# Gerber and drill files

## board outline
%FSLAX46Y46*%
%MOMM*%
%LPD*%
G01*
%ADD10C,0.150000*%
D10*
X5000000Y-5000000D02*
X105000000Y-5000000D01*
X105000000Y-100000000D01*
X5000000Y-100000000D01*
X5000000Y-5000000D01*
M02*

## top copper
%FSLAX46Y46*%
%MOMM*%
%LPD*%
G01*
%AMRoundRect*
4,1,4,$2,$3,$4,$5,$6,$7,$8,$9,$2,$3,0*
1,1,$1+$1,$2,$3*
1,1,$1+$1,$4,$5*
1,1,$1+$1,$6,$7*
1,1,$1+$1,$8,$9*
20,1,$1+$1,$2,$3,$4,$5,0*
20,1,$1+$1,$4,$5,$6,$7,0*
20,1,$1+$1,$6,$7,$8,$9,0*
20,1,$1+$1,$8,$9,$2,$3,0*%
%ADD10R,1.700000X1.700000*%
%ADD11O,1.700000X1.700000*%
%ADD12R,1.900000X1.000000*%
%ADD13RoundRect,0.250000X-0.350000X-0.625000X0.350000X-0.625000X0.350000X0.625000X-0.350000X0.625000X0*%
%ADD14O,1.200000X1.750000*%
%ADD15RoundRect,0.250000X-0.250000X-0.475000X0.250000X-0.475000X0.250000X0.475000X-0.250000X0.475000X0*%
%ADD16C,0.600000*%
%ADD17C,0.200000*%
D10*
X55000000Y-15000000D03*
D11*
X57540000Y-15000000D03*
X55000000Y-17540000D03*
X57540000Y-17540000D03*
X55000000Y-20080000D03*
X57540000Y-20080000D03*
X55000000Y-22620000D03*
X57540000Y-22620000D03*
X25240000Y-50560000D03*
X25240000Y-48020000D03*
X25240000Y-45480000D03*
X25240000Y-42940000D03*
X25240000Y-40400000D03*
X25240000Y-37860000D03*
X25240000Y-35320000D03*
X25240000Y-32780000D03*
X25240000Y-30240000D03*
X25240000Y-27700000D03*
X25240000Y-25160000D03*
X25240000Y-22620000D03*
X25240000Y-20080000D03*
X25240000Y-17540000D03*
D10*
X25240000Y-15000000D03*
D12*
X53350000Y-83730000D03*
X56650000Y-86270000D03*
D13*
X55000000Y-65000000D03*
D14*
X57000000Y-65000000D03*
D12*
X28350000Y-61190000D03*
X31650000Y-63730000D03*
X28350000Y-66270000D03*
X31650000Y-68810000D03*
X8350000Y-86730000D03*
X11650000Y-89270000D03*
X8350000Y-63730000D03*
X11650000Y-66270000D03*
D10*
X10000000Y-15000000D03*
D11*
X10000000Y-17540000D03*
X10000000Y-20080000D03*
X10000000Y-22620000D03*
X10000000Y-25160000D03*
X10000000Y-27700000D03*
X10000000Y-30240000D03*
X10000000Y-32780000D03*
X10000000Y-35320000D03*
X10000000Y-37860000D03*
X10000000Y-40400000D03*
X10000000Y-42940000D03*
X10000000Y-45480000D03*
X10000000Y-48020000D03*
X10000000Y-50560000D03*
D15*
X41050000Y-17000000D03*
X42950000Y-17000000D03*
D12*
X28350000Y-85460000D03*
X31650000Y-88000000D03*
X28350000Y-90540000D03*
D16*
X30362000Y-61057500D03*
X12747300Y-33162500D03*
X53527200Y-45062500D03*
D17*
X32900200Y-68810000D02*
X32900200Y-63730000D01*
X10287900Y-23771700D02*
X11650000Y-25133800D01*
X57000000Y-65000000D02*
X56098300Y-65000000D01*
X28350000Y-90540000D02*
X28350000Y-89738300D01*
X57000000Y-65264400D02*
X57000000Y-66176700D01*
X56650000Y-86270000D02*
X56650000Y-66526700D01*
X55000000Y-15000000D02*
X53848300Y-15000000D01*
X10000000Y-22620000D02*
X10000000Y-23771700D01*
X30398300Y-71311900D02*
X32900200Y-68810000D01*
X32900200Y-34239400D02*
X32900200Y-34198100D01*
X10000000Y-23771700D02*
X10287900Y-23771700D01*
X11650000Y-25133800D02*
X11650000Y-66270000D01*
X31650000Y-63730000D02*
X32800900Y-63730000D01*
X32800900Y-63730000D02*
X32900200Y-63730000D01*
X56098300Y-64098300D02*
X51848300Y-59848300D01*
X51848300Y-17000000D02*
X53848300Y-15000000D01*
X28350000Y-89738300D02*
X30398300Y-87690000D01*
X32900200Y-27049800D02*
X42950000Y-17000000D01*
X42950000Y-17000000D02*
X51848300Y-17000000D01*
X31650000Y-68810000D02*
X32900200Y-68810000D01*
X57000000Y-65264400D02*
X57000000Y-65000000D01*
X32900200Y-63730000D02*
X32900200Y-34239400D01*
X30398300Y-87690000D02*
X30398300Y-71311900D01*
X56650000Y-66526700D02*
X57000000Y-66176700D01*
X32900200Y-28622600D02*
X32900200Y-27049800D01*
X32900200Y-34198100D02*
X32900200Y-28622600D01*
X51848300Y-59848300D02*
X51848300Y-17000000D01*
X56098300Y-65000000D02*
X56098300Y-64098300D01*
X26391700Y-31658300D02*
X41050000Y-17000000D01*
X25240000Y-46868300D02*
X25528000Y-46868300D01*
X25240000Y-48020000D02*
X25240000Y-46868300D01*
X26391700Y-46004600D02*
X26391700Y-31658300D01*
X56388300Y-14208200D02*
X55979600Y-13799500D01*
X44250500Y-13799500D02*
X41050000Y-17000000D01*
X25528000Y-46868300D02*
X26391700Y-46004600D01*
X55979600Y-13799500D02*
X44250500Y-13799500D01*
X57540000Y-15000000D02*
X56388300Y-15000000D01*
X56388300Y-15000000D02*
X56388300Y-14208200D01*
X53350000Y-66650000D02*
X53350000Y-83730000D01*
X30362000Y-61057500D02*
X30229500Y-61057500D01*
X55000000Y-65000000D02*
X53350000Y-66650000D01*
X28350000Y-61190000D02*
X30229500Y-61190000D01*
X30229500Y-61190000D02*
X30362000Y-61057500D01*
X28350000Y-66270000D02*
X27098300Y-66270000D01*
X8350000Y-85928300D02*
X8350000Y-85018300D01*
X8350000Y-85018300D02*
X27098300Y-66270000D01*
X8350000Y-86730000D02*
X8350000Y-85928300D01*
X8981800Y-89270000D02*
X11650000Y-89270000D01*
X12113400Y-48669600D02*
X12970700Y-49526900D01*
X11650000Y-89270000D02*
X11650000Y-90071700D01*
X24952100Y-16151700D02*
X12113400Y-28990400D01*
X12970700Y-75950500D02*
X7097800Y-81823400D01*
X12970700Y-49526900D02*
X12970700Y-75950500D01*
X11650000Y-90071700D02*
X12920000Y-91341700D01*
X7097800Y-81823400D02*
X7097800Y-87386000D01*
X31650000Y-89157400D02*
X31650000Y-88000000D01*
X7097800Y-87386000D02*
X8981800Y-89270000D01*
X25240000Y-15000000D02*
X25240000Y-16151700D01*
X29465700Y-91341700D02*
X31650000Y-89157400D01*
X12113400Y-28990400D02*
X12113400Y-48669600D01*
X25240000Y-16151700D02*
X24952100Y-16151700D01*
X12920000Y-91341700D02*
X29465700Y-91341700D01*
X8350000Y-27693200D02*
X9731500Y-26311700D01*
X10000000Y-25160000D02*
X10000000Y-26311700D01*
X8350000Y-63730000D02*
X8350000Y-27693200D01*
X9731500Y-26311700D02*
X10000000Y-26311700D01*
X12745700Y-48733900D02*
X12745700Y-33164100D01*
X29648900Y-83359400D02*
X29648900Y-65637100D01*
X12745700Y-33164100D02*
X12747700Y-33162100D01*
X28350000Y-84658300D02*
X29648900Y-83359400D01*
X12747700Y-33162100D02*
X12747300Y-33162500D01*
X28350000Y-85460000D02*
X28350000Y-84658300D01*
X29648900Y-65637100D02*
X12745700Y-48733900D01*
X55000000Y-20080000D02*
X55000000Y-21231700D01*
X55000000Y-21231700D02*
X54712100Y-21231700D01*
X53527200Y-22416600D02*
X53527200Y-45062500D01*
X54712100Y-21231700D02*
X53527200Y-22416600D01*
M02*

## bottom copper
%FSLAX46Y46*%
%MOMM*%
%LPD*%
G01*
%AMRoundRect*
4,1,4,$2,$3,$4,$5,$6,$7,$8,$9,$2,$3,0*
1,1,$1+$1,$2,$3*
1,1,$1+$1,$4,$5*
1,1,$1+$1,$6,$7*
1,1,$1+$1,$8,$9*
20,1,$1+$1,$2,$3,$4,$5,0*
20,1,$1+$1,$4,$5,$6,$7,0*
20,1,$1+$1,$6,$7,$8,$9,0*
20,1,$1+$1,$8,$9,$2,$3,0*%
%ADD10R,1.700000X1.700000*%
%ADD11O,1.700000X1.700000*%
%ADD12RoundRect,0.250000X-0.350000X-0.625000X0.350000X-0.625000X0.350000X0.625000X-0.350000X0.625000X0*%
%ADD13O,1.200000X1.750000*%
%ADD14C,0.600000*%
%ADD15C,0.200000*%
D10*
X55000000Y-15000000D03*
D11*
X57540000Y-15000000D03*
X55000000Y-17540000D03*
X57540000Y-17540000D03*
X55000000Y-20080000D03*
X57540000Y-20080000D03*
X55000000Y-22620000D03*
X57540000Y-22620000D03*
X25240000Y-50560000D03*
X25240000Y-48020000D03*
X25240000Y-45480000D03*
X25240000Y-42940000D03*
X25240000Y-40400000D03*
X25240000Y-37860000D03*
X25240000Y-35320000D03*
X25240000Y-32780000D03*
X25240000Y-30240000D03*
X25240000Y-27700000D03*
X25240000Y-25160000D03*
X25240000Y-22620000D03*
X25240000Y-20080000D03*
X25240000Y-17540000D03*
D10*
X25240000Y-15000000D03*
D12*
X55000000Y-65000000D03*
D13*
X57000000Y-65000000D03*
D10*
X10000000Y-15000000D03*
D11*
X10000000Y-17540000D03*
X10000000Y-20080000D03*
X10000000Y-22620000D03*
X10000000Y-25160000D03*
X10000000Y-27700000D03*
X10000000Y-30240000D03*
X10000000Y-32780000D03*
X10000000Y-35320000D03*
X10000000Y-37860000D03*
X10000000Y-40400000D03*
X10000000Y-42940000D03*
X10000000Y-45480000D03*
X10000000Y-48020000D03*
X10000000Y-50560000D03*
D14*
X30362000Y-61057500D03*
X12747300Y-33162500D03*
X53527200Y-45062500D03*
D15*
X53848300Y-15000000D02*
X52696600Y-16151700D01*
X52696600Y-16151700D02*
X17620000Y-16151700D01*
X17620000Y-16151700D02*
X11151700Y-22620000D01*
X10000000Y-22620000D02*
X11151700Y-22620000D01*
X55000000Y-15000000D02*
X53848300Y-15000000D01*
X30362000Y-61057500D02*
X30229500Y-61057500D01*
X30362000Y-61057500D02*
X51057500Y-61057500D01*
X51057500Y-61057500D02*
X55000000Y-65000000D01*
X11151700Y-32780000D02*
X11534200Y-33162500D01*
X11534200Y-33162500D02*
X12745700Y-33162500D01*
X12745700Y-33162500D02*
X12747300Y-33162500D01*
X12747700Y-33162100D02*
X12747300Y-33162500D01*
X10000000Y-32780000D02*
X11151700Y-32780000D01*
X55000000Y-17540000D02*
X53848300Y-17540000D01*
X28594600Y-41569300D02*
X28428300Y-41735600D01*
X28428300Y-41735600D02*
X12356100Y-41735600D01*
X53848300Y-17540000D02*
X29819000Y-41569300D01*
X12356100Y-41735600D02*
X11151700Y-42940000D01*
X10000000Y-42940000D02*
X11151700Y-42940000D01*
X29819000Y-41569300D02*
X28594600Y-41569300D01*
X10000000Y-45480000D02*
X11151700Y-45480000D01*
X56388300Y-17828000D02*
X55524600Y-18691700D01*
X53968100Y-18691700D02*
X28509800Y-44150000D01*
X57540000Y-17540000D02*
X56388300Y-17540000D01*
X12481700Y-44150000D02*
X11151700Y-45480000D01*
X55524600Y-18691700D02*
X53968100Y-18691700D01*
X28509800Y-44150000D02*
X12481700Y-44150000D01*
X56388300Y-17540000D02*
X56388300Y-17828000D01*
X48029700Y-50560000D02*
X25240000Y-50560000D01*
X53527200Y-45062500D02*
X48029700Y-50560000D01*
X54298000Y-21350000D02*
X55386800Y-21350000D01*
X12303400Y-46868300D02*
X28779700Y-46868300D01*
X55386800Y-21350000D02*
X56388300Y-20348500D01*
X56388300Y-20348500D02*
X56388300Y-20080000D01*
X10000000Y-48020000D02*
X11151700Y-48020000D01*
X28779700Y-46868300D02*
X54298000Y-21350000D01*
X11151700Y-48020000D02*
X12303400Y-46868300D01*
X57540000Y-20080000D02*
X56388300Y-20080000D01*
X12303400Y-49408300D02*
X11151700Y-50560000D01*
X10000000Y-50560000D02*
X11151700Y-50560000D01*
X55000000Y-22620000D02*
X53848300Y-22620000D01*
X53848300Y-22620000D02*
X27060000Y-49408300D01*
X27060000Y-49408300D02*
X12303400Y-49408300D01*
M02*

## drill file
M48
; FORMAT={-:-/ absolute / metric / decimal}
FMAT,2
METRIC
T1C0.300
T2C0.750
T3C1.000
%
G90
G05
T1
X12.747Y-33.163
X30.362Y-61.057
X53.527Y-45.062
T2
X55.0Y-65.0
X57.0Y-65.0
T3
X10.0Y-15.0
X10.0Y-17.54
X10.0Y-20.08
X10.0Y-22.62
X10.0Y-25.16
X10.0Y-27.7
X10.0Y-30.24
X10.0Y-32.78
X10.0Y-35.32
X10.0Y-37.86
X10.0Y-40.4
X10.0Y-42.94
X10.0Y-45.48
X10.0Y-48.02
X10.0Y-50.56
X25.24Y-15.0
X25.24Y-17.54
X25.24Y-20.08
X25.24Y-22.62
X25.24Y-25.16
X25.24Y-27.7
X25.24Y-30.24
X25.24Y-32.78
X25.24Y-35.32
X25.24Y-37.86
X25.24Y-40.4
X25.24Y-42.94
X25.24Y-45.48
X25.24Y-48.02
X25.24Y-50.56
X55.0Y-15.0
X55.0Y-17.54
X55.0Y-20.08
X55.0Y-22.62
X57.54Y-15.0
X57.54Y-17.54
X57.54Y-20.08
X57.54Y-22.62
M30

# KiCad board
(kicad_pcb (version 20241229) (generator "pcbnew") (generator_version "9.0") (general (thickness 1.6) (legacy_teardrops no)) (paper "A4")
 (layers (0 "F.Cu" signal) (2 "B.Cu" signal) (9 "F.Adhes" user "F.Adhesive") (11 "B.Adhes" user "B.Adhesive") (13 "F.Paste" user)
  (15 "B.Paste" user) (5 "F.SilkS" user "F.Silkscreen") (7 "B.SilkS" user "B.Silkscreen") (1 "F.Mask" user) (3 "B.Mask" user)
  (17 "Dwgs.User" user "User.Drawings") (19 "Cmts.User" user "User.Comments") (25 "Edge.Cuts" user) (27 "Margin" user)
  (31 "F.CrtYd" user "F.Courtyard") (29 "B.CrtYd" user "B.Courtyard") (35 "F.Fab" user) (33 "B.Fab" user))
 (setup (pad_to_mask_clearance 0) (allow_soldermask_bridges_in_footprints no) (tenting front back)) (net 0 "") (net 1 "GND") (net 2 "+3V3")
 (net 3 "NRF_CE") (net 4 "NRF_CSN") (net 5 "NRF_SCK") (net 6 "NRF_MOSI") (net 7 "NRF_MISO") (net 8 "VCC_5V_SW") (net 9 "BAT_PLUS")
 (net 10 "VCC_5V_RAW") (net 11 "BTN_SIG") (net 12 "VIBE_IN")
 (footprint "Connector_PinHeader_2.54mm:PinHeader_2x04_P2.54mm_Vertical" (layer "F.Cu") (at 55 15)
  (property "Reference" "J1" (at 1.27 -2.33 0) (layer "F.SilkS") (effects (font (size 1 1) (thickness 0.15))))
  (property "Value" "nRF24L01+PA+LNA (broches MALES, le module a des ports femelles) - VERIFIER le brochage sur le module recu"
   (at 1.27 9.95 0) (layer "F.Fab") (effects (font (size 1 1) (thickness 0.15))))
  (pad "1" thru_hole rect (at 0 0) (size 1.7 1.7) (drill 1) (layers "*.Cu" "*.Mask") (remove_unused_layers no) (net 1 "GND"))
  (pad "2" thru_hole oval (at 2.54 0) (size 1.7 1.7) (drill 1) (layers "*.Cu" "*.Mask") (remove_unused_layers no) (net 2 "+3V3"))
  (pad "3" thru_hole oval (at 0 2.54) (size 1.7 1.7) (drill 1) (layers "*.Cu" "*.Mask") (remove_unused_layers no) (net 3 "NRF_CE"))
  (pad "4" thru_hole oval (at 2.54 2.54) (size 1.7 1.7) (drill 1) (layers "*.Cu" "*.Mask") (remove_unused_layers no) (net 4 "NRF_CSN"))
  (pad "5" thru_hole oval (at 0 5.08) (size 1.7 1.7) (drill 1) (layers "*.Cu" "*.Mask") (remove_unused_layers no) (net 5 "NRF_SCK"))
  (pad "6" thru_hole oval (at 2.54 5.08) (size 1.7 1.7) (drill 1) (layers "*.Cu" "*.Mask") (remove_unused_layers no) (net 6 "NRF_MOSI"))
  (pad "7" thru_hole oval (at 0 7.62) (size 1.7 1.7) (drill 1) (layers "*.Cu" "*.Mask") (remove_unused_layers no) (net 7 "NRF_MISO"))
  (pad "8" thru_hole oval (at 2.54 7.62) (size 1.7 1.7) (drill 1) (layers "*.Cu" "*.Mask") (remove_unused_layers no)))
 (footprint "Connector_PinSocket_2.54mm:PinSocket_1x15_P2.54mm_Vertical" (layer "F.Cu") (at 25.24 15)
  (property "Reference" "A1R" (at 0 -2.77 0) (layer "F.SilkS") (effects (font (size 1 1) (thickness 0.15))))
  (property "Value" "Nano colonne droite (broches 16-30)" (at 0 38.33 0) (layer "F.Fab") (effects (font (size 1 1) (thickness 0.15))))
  (pad "16" thru_hole oval (at 0 35.56) (size 1.7 1.7) (drill 1) (layers "*.Cu" "*.Mask") (remove_unused_layers no) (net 5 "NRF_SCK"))
  (pad "17" thru_hole oval (at 0 33.02) (size 1.7 1.7) (drill 1) (layers "*.Cu" "*.Mask") (remove_unused_layers no) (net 2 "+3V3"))
  (pad "18" thru_hole oval (at 0 30.48) (size 1.7 1.7) (drill 1) (layers "*.Cu" "*.Mask") (remove_unused_layers no))
  (pad "19" thru_hole oval (at 0 27.94) (size 1.7 1.7) (drill 1) (layers "*.Cu" "*.Mask") (remove_unused_layers no))
  (pad "20" thru_hole oval (at 0 25.4) (size 1.7 1.7) (drill 1) (layers "*.Cu" "*.Mask") (remove_unused_layers no))
  (pad "21" thru_hole oval (at 0 22.86) (size 1.7 1.7) (drill 1) (layers "*.Cu" "*.Mask") (remove_unused_layers no))
  (pad "22" thru_hole oval (at 0 20.32) (size 1.7 1.7) (drill 1) (layers "*.Cu" "*.Mask") (remove_unused_layers no))
  (pad "23" thru_hole oval (at 0 17.78) (size 1.7 1.7) (drill 1) (layers "*.Cu" "*.Mask") (remove_unused_layers no))
  (pad "24" thru_hole oval (at 0 15.24) (size 1.7 1.7) (drill 1) (layers "*.Cu" "*.Mask") (remove_unused_layers no))
  (pad "25" thru_hole oval (at 0 12.7) (size 1.7 1.7) (drill 1) (layers "*.Cu" "*.Mask") (remove_unused_layers no))
  (pad "26" thru_hole oval (at 0 10.16) (size 1.7 1.7) (drill 1) (layers "*.Cu" "*.Mask") (remove_unused_layers no))
  (pad "27" thru_hole oval (at 0 7.62) (size 1.7 1.7) (drill 1) (layers "*.Cu" "*.Mask") (remove_unused_layers no))
  (pad "28" thru_hole oval (at 0 5.08) (size 1.7 1.7) (drill 1) (layers "*.Cu" "*.Mask") (remove_unused_layers no))
  (pad "29" thru_hole oval (at 0 2.54) (size 1.7 1.7) (drill 1) (layers "*.Cu" "*.Mask") (remove_unused_layers no))
  (pad "30" thru_hole rect (at 0 0) (size 1.7 1.7) (drill 1) (layers "*.Cu" "*.Mask") (remove_unused_layers no) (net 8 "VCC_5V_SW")))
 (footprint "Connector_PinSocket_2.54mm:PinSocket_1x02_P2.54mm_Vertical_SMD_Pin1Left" (layer "F.Cu") (at 55 85)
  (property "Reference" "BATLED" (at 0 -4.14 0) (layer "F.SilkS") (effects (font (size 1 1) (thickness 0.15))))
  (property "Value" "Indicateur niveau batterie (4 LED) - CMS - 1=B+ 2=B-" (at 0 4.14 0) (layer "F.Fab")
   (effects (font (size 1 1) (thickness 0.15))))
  (pad "1" smd rect (at -1.65 -1.27) (size 1.9 1) (layers "F.Cu" "F.Mask" "F.Paste") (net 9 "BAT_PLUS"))
  (pad "2" smd rect (at 1.65 1.27) (size 1.9 1) (layers "F.Cu" "F.Mask" "F.Paste") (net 1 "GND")))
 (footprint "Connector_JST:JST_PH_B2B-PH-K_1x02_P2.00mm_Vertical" (layer "F.Cu") (at 55 65)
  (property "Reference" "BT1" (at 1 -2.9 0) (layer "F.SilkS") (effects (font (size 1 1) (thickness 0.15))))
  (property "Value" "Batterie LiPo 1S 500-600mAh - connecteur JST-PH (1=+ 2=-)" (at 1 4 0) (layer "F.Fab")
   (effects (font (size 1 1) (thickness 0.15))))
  (pad "1" thru_hole roundrect (at 0 0) (size 1.2 1.75) (drill 0.75) (layers "*.Cu" "*.Mask") (remove_unused_layers no)
   (roundrect_rratio 0.208333) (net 9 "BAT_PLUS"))
  (pad "2" thru_hole oval (at 2 0) (size 1.2 1.75) (drill 0.75) (layers "*.Cu" "*.Mask") (remove_unused_layers no) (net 1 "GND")))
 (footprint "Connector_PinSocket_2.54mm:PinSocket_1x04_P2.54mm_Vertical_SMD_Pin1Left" (layer "F.Cu") (at 30 65)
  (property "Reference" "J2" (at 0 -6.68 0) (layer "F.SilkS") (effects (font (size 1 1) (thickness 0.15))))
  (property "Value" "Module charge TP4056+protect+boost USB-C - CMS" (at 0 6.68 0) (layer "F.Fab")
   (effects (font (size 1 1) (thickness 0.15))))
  (pad "1" smd rect (at -1.65 -3.81) (size 1.9 1) (layers "F.Cu" "F.Mask" "F.Paste") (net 9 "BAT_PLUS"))
  (pad "2" smd rect (at 1.65 -1.27) (size 1.9 1) (layers "F.Cu" "F.Mask" "F.Paste") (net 1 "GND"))
  (pad "3" smd rect (at -1.65 1.27) (size 1.9 1) (layers "F.Cu" "F.Mask" "F.Paste") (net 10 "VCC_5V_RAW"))
  (pad "4" smd rect (at 1.65 3.81) (size 1.9 1) (layers "F.Cu" "F.Mask" "F.Paste") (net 1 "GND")))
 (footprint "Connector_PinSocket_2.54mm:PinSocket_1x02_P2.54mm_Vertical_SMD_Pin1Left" (layer "F.Cu") (at 10 88)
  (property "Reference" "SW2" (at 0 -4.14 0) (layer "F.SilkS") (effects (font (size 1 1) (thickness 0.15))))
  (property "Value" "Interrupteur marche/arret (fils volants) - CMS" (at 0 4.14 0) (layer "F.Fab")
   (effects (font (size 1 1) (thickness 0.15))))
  (pad "1" smd rect (at -1.65 -1.27) (size 1.9 1) (layers "F.Cu" "F.Mask" "F.Paste") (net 10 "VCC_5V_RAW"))
  (pad "2" smd rect (at 1.65 1.27) (size 1.9 1) (layers "F.Cu" "F.Mask" "F.Paste") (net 8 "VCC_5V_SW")))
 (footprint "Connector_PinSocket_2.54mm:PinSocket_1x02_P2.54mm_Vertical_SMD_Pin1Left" (layer "F.Cu") (at 10 65)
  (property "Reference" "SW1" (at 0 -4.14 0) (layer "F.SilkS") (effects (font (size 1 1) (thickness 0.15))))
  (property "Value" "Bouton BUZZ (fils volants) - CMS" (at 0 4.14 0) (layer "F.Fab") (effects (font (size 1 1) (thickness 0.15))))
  (pad "1" smd rect (at -1.65 -1.27) (size 1.9 1) (layers "F.Cu" "F.Mask" "F.Paste") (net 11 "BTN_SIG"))
  (pad "2" smd rect (at 1.65 1.27) (size 1.9 1) (layers "F.Cu" "F.Mask" "F.Paste") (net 1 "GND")))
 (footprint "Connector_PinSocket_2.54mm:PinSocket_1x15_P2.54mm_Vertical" (layer "F.Cu") (at 10 15)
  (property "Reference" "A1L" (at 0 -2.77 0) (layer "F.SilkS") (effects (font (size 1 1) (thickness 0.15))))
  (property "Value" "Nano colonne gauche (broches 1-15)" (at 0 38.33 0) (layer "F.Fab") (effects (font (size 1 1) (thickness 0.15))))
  (pad "1" thru_hole rect (at 0 0) (size 1.7 1.7) (drill 1) (layers "*.Cu" "*.Mask") (remove_unused_layers no))
  (pad "2" thru_hole oval (at 0 2.54) (size 1.7 1.7) (drill 1) (layers "*.Cu" "*.Mask") (remove_unused_layers no))
  (pad "3" thru_hole oval (at 0 5.08) (size 1.7 1.7) (drill 1) (layers "*.Cu" "*.Mask") (remove_unused_layers no))
  (pad "4" thru_hole oval (at 0 7.62) (size 1.7 1.7) (drill 1) (layers "*.Cu" "*.Mask") (remove_unused_layers no) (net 1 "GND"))
  (pad "5" thru_hole oval (at 0 10.16) (size 1.7 1.7) (drill 1) (layers "*.Cu" "*.Mask") (remove_unused_layers no) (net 11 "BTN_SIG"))
  (pad "6" thru_hole oval (at 0 12.7) (size 1.7 1.7) (drill 1) (layers "*.Cu" "*.Mask") (remove_unused_layers no))
  (pad "7" thru_hole oval (at 0 15.24) (size 1.7 1.7) (drill 1) (layers "*.Cu" "*.Mask") (remove_unused_layers no))
  (pad "8" thru_hole oval (at 0 17.78) (size 1.7 1.7) (drill 1) (layers "*.Cu" "*.Mask") (remove_unused_layers no) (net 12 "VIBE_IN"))
  (pad "9" thru_hole oval (at 0 20.32) (size 1.7 1.7) (drill 1) (layers "*.Cu" "*.Mask") (remove_unused_layers no))
  (pad "10" thru_hole oval (at 0 22.86) (size 1.7 1.7) (drill 1) (layers "*.Cu" "*.Mask") (remove_unused_layers no))
  (pad "11" thru_hole oval (at 0 25.4) (size 1.7 1.7) (drill 1) (layers "*.Cu" "*.Mask") (remove_unused_layers no))
  (pad "12" thru_hole oval (at 0 27.94) (size 1.7 1.7) (drill 1) (layers "*.Cu" "*.Mask") (remove_unused_layers no) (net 3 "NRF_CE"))
  (pad "13" thru_hole oval (at 0 30.48) (size 1.7 1.7) (drill 1) (layers "*.Cu" "*.Mask") (remove_unused_layers no) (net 4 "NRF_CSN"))
  (pad "14" thru_hole oval (at 0 33.02) (size 1.7 1.7) (drill 1) (layers "*.Cu" "*.Mask") (remove_unused_layers no) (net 6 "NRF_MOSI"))
  (pad "15" thru_hole oval (at 0 35.56) (size 1.7 1.7) (drill 1) (layers "*.Cu" "*.Mask") (remove_unused_layers no) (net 7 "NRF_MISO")))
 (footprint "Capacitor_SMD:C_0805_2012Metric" (layer "F.Cu") (at 42 17)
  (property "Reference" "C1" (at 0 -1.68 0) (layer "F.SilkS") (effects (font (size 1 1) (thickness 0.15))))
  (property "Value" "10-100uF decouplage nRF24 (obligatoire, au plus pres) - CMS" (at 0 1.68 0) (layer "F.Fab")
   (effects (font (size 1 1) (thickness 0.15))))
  (pad "1" smd roundrect (at -0.95 0) (size 1 1.45) (layers "F.Cu" "F.Mask" "F.Paste") (roundrect_rratio 0.25) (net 2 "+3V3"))
  (pad "2" smd roundrect (at 0.95 0) (size 1 1.45) (layers "F.Cu" "F.Mask" "F.Paste") (roundrect_rratio 0.25) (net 1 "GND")))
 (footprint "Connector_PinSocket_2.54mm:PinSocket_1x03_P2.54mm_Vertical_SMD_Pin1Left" (layer "F.Cu") (at 30 88)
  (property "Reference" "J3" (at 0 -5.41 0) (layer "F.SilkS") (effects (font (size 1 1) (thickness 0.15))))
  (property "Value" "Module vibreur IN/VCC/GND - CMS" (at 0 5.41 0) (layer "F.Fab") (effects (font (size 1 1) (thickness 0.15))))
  (pad "1" smd rect (at -1.65 -2.54) (size 1.9 1) (layers "F.Cu" "F.Mask" "F.Paste") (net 12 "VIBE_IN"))
  (pad "2" smd rect (at 1.65 0) (size 1.9 1) (layers "F.Cu" "F.Mask" "F.Paste") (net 8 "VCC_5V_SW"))
  (pad "3" smd rect (at -1.65 2.54) (size 1.9 1) (layers "F.Cu" "F.Mask" "F.Paste") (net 1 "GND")))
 (gr_rect (start 5 5) (end 105 100) (stroke (width 0.15) (type default)) (fill no) (layer "Edge.Cuts"))
 (segment (start 32.9002 68.81) (end 32.9002 63.73) (width 0.2) (layer "F.Cu") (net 1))
 (segment (start 10.2879 23.7717) (end 11.65 25.1338) (width 0.2) (layer "F.Cu") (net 1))
 (segment (start 57 65) (end 56.0983 65) (width 0.2) (layer "F.Cu") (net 1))
 (segment (start 28.35 90.54) (end 28.35 89.7383) (width 0.2) (layer "F.Cu") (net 1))
 (segment (start 57 65.2644) (end 57 66.1767) (width 0.2) (layer "F.Cu") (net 1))
 (segment (start 56.65 86.27) (end 56.65 66.5267) (width 0.2) (layer "F.Cu") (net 1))
 (segment (start 55 15) (end 53.8483 15) (width 0.2) (layer "F.Cu") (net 1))
 (segment (start 10 22.62) (end 10 23.7717) (width 0.2) (layer "F.Cu") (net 1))
 (segment (start 30.3983 71.3119) (end 32.9002 68.81) (width 0.2) (layer "F.Cu") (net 1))
 (segment (start 32.9002 34.2394) (end 32.9002 34.1981) (width 0.2) (layer "F.Cu") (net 1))
 (segment (start 10 23.7717) (end 10.2879 23.7717) (width 0.2) (layer "F.Cu") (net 1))
 (segment (start 11.65 25.1338) (end 11.65 66.27) (width 0.2) (layer "F.Cu") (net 1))
 (segment (start 31.65 63.73) (end 32.8009 63.73) (width 0.2) (layer "F.Cu") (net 1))
 (segment (start 32.8009 63.73) (end 32.9002 63.73) (width 0.2) (layer "F.Cu") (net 1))
 (segment (start 56.0983 64.0983) (end 51.8483 59.8483) (width 0.2) (layer "F.Cu") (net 1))
 (segment (start 51.8483 17) (end 53.8483 15) (width 0.2) (layer "F.Cu") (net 1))
 (segment (start 28.35 89.7383) (end 30.3983 87.69) (width 0.2) (layer "F.Cu") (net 1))
 (segment (start 32.9002 27.0498) (end 42.95 17) (width 0.2) (layer "F.Cu") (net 1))
 (segment (start 42.95 17) (end 51.8483 17) (width 0.2) (layer "F.Cu") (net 1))
 (segment (start 31.65 68.81) (end 32.9002 68.81) (width 0.2) (layer "F.Cu") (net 1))
 (segment (start 57 65.2644) (end 57 65) (width 0.2) (layer "F.Cu") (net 1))
 (segment (start 32.9002 63.73) (end 32.9002 34.2394) (width 0.2) (layer "F.Cu") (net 1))
 (segment (start 30.3983 87.69) (end 30.3983 71.3119) (width 0.2) (layer "F.Cu") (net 1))
 (segment (start 56.65 66.5267) (end 57 66.1767) (width 0.2) (layer "F.Cu") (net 1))
 (segment (start 32.9002 28.6226) (end 32.9002 27.0498) (width 0.2) (layer "F.Cu") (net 1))
 (segment (start 32.9002 34.1981) (end 32.9002 28.6226) (width 0.2) (layer "F.Cu") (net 1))
 (segment (start 51.8483 59.8483) (end 51.8483 17) (width 0.2) (layer "F.Cu") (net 1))
 (segment (start 56.0983 65) (end 56.0983 64.0983) (width 0.2) (layer "F.Cu") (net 1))
 (segment (start 53.8483 15) (end 52.6966 16.1517) (width 0.2) (layer "B.Cu") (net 1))
 (segment (start 52.6966 16.1517) (end 17.62 16.1517) (width 0.2) (layer "B.Cu") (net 1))
 (segment (start 17.62 16.1517) (end 11.1517 22.62) (width 0.2) (layer "B.Cu") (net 1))
 (segment (start 10 22.62) (end 11.1517 22.62) (width 0.2) (layer "B.Cu") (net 1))
 (segment (start 55 15) (end 53.8483 15) (width 0.2) (layer "B.Cu") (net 1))
 (segment (start 26.3917 31.6583) (end 41.05 17) (width 0.2) (layer "F.Cu") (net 2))
 (segment (start 25.24 46.8683) (end 25.528 46.8683) (width 0.2) (layer "F.Cu") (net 2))
 (segment (start 25.24 48.02) (end 25.24 46.8683) (width 0.2) (layer "F.Cu") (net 2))
 (segment (start 26.3917 46.0046) (end 26.3917 31.6583) (width 0.2) (layer "F.Cu") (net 2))
 (segment (start 56.3883 14.2082) (end 55.9796 13.7995) (width 0.2) (layer "F.Cu") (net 2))
 (segment (start 44.2505 13.7995) (end 41.05 17) (width 0.2) (layer "F.Cu") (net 2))
 (segment (start 25.528 46.8683) (end 26.3917 46.0046) (width 0.2) (layer "F.Cu") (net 2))
 (segment (start 55.9796 13.7995) (end 44.2505 13.7995) (width 0.2) (layer "F.Cu") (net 2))
 (segment (start 57.54 15) (end 56.3883 15) (width 0.2) (layer "F.Cu") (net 2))
 (segment (start 56.3883 15) (end 56.3883 14.2082) (width 0.2) (layer "F.Cu") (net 2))
 (segment (start 53.35 66.65) (end 53.35 83.73) (width 0.2) (layer "F.Cu") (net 9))
 (segment (start 30.362 61.0575) (end 30.2295 61.0575) (width 0.2) (layer "F.Cu") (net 9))
 (segment (start 55 65) (end 53.35 66.65) (width 0.2) (layer "F.Cu") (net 9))
 (segment (start 28.35 61.19) (end 30.2295 61.19) (width 0.2) (layer "F.Cu") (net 9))
 (segment (start 30.2295 61.19) (end 30.362 61.0575) (width 0.2) (layer "F.Cu") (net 9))
 (via (at 30.362 61.0575) (size 0.6) (drill 0.3) (layers "F.Cu" "B.Cu") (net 9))
 (segment (start 30.362 61.0575) (end 30.2295 61.0575) (width 0.2) (layer "B.Cu") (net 9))
 (segment (start 30.362 61.0575) (end 51.0575 61.0575) (width 0.2) (layer "B.Cu") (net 9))
 (segment (start 51.0575 61.0575) (end 55 65) (width 0.2) (layer "B.Cu") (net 9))
 (segment (start 28.35 66.27) (end 27.0983 66.27) (width 0.2) (layer "F.Cu") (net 10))
 (segment (start 8.35 85.9283) (end 8.35 85.0183) (width 0.2) (layer "F.Cu") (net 10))
 (segment (start 8.35 85.0183) (end 27.0983 66.27) (width 0.2) (layer "F.Cu") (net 10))
 (segment (start 8.35 86.73) (end 8.35 85.9283) (width 0.2) (layer "F.Cu") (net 10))
 (segment (start 8.9818 89.27) (end 11.65 89.27) (width 0.2) (layer "F.Cu") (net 8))
 (segment (start 12.1134 48.6696) (end 12.9707 49.5269) (width 0.2) (layer "F.Cu") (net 8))
 (segment (start 11.65 89.27) (end 11.65 90.0717) (width 0.2) (layer "F.Cu") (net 8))
 (segment (start 24.9521 16.1517) (end 12.1134 28.9904) (width 0.2) (layer "F.Cu") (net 8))
 (segment (start 12.9707 75.9505) (end 7.0978 81.8234) (width 0.2) (layer "F.Cu") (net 8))
 (segment (start 12.9707 49.5269) (end 12.9707 75.9505) (width 0.2) (layer "F.Cu") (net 8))
 (segment (start 11.65 90.0717) (end 12.92 91.3417) (width 0.2) (layer "F.Cu") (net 8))
 (segment (start 7.0978 81.8234) (end 7.0978 87.386) (width 0.2) (layer "F.Cu") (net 8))
 (segment (start 31.65 89.1574) (end 31.65 88) (width 0.2) (layer "F.Cu") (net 8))
 (segment (start 7.0978 87.386) (end 8.9818 89.27) (width 0.2) (layer "F.Cu") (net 8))
 (segment (start 25.24 15) (end 25.24 16.1517) (width 0.2) (layer "F.Cu") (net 8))
 (segment (start 29.4657 91.3417) (end 31.65 89.1574) (width 0.2) (layer "F.Cu") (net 8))
 (segment (start 12.1134 28.9904) (end 12.1134 48.6696) (width 0.2) (layer "F.Cu") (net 8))
 (segment (start 25.24 16.1517) (end 24.9521 16.1517) (width 0.2) (layer "F.Cu") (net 8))
 (segment (start 12.92 91.3417) (end 29.4657 91.3417) (width 0.2) (layer "F.Cu") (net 8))
 (segment (start 8.35 27.6932) (end 9.7315 26.3117) (width 0.2) (layer "F.Cu") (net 11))
 (segment (start 10 25.16) (end 10 26.3117) (width 0.2) (layer "F.Cu") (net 11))
 (segment (start 8.35 63.73) (end 8.35 27.6932) (width 0.2) (layer "F.Cu") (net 11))
 (segment (start 9.7315 26.3117) (end 10 26.3117) (width 0.2) (layer "F.Cu") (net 11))
 (segment (start 12.7457 48.7339) (end 12.7457 33.1641) (width 0.2) (layer "F.Cu") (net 12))
 (segment (start 29.6489 83.3594) (end 29.6489 65.6371) (width 0.2) (layer "F.Cu") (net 12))
 (segment (start 12.7457 33.1641) (end 12.7477 33.1621) (width 0.2) (layer "F.Cu") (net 12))
 (segment (start 28.35 84.6583) (end 29.6489 83.3594) (width 0.2) (layer "F.Cu") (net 12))
 (segment (start 12.7477 33.1621) (end 12.7473 33.1625) (width 0.2) (layer "F.Cu") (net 12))
 (segment (start 28.35 85.46) (end 28.35 84.6583) (width 0.2) (layer "F.Cu") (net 12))
 (segment (start 29.6489 65.6371) (end 12.7457 48.7339) (width 0.2) (layer "F.Cu") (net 12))
 (via (at 12.7473 33.1625) (size 0.6) (drill 0.3) (layers "F.Cu" "B.Cu") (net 12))
 (segment (start 11.1517 32.78) (end 11.5342 33.1625) (width 0.2) (layer "B.Cu") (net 12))
 (segment (start 11.5342 33.1625) (end 12.7457 33.1625) (width 0.2) (layer "B.Cu") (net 12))
 (segment (start 12.7457 33.1625) (end 12.7473 33.1625) (width 0.2) (layer "B.Cu") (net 12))
 (segment (start 12.7477 33.1621) (end 12.7473 33.1625) (width 0.2) (layer "B.Cu") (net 12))
 (segment (start 10 32.78) (end 11.1517 32.78) (width 0.2) (layer "B.Cu") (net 12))
 (segment (start 55 17.54) (end 53.8483 17.54) (width 0.2) (layer "B.Cu") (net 3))
 (segment (start 28.5946 41.5693) (end 28.4283 41.7356) (width 0.2) (layer "B.Cu") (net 3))
 (segment (start 28.4283 41.7356) (end 12.3561 41.7356) (width 0.2) (layer "B.Cu") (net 3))
 (segment (start 53.8483 17.54) (end 29.819 41.5693) (width 0.2) (layer "B.Cu") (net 3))
 (segment (start 12.3561 41.7356) (end 11.1517 42.94) (width 0.2) (layer "B.Cu") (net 3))
 (segment (start 10 42.94) (end 11.1517 42.94) (width 0.2) (layer "B.Cu") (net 3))
 (segment (start 29.819 41.5693) (end 28.5946 41.5693) (width 0.2) (layer "B.Cu") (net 3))
 (segment (start 10 45.48) (end 11.1517 45.48) (width 0.2) (layer "B.Cu") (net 4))
 (segment (start 56.3883 17.828) (end 55.5246 18.6917) (width 0.2) (layer "B.Cu") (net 4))
 (segment (start 53.9681 18.6917) (end 28.5098 44.15) (width 0.2) (layer "B.Cu") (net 4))
 (segment (start 57.54 17.54) (end 56.3883 17.54) (width 0.2) (layer "B.Cu") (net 4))
 (segment (start 12.4817 44.15) (end 11.1517 45.48) (width 0.2) (layer "B.Cu") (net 4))
 (segment (start 55.5246 18.6917) (end 53.9681 18.6917) (width 0.2) (layer "B.Cu") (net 4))
 (segment (start 28.5098 44.15) (end 12.4817 44.15) (width 0.2) (layer "B.Cu") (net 4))
 (segment (start 56.3883 17.54) (end 56.3883 17.828) (width 0.2) (layer "B.Cu") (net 4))
 (segment (start 55 20.08) (end 55 21.2317) (width 0.2) (layer "F.Cu") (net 5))
 (segment (start 55 21.2317) (end 54.7121 21.2317) (width 0.2) (layer "F.Cu") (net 5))
 (segment (start 53.5272 22.4166) (end 53.5272 45.0625) (width 0.2) (layer "F.Cu") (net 5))
 (segment (start 54.7121 21.2317) (end 53.5272 22.4166) (width 0.2) (layer "F.Cu") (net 5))
 (via (at 53.5272 45.0625) (size 0.6) (drill 0.3) (layers "F.Cu" "B.Cu") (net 5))
 (segment (start 48.0297 50.56) (end 25.24 50.56) (width 0.2) (layer "B.Cu") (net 5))
 (segment (start 53.5272 45.0625) (end 48.0297 50.56) (width 0.2) (layer "B.Cu") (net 5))
 (segment (start 54.298 21.35) (end 55.3868 21.35) (width 0.2) (layer "B.Cu") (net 6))
 (segment (start 12.3034 46.8683) (end 28.7797 46.8683) (width 0.2) (layer "B.Cu") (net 6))
 (segment (start 55.3868 21.35) (end 56.3883 20.3485) (width 0.2) (layer "B.Cu") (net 6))
 (segment (start 56.3883 20.3485) (end 56.3883 20.08) (width 0.2) (layer "B.Cu") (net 6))
 (segment (start 10 48.02) (end 11.1517 48.02) (width 0.2) (layer "B.Cu") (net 6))
 (segment (start 28.7797 46.8683) (end 54.298 21.35) (width 0.2) (layer "B.Cu") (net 6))
 (segment (start 11.1517 48.02) (end 12.3034 46.8683) (width 0.2) (layer "B.Cu") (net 6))
 (segment (start 57.54 20.08) (end 56.3883 20.08) (width 0.2) (layer "B.Cu") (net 6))
 (segment (start 12.3034 49.4083) (end 11.1517 50.56) (width 0.2) (layer "B.Cu") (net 7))
 (segment (start 10 50.56) (end 11.1517 50.56) (width 0.2) (layer "B.Cu") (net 7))
 (segment (start 55 22.62) (end 53.8483 22.62) (width 0.2) (layer "B.Cu") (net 7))
 (segment (start 53.8483 22.62) (end 27.06 49.4083) (width 0.2) (layer "B.Cu") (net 7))
 (segment (start 27.06 49.4083) (end 12.3034 49.4083) (width 0.2) (layer "B.Cu") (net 7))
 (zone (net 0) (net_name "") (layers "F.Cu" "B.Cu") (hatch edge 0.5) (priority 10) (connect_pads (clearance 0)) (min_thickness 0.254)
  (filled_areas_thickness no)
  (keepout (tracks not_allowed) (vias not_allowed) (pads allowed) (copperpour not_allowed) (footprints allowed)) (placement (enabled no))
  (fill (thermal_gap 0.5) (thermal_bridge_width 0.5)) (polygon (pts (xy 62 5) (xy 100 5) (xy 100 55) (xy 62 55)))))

